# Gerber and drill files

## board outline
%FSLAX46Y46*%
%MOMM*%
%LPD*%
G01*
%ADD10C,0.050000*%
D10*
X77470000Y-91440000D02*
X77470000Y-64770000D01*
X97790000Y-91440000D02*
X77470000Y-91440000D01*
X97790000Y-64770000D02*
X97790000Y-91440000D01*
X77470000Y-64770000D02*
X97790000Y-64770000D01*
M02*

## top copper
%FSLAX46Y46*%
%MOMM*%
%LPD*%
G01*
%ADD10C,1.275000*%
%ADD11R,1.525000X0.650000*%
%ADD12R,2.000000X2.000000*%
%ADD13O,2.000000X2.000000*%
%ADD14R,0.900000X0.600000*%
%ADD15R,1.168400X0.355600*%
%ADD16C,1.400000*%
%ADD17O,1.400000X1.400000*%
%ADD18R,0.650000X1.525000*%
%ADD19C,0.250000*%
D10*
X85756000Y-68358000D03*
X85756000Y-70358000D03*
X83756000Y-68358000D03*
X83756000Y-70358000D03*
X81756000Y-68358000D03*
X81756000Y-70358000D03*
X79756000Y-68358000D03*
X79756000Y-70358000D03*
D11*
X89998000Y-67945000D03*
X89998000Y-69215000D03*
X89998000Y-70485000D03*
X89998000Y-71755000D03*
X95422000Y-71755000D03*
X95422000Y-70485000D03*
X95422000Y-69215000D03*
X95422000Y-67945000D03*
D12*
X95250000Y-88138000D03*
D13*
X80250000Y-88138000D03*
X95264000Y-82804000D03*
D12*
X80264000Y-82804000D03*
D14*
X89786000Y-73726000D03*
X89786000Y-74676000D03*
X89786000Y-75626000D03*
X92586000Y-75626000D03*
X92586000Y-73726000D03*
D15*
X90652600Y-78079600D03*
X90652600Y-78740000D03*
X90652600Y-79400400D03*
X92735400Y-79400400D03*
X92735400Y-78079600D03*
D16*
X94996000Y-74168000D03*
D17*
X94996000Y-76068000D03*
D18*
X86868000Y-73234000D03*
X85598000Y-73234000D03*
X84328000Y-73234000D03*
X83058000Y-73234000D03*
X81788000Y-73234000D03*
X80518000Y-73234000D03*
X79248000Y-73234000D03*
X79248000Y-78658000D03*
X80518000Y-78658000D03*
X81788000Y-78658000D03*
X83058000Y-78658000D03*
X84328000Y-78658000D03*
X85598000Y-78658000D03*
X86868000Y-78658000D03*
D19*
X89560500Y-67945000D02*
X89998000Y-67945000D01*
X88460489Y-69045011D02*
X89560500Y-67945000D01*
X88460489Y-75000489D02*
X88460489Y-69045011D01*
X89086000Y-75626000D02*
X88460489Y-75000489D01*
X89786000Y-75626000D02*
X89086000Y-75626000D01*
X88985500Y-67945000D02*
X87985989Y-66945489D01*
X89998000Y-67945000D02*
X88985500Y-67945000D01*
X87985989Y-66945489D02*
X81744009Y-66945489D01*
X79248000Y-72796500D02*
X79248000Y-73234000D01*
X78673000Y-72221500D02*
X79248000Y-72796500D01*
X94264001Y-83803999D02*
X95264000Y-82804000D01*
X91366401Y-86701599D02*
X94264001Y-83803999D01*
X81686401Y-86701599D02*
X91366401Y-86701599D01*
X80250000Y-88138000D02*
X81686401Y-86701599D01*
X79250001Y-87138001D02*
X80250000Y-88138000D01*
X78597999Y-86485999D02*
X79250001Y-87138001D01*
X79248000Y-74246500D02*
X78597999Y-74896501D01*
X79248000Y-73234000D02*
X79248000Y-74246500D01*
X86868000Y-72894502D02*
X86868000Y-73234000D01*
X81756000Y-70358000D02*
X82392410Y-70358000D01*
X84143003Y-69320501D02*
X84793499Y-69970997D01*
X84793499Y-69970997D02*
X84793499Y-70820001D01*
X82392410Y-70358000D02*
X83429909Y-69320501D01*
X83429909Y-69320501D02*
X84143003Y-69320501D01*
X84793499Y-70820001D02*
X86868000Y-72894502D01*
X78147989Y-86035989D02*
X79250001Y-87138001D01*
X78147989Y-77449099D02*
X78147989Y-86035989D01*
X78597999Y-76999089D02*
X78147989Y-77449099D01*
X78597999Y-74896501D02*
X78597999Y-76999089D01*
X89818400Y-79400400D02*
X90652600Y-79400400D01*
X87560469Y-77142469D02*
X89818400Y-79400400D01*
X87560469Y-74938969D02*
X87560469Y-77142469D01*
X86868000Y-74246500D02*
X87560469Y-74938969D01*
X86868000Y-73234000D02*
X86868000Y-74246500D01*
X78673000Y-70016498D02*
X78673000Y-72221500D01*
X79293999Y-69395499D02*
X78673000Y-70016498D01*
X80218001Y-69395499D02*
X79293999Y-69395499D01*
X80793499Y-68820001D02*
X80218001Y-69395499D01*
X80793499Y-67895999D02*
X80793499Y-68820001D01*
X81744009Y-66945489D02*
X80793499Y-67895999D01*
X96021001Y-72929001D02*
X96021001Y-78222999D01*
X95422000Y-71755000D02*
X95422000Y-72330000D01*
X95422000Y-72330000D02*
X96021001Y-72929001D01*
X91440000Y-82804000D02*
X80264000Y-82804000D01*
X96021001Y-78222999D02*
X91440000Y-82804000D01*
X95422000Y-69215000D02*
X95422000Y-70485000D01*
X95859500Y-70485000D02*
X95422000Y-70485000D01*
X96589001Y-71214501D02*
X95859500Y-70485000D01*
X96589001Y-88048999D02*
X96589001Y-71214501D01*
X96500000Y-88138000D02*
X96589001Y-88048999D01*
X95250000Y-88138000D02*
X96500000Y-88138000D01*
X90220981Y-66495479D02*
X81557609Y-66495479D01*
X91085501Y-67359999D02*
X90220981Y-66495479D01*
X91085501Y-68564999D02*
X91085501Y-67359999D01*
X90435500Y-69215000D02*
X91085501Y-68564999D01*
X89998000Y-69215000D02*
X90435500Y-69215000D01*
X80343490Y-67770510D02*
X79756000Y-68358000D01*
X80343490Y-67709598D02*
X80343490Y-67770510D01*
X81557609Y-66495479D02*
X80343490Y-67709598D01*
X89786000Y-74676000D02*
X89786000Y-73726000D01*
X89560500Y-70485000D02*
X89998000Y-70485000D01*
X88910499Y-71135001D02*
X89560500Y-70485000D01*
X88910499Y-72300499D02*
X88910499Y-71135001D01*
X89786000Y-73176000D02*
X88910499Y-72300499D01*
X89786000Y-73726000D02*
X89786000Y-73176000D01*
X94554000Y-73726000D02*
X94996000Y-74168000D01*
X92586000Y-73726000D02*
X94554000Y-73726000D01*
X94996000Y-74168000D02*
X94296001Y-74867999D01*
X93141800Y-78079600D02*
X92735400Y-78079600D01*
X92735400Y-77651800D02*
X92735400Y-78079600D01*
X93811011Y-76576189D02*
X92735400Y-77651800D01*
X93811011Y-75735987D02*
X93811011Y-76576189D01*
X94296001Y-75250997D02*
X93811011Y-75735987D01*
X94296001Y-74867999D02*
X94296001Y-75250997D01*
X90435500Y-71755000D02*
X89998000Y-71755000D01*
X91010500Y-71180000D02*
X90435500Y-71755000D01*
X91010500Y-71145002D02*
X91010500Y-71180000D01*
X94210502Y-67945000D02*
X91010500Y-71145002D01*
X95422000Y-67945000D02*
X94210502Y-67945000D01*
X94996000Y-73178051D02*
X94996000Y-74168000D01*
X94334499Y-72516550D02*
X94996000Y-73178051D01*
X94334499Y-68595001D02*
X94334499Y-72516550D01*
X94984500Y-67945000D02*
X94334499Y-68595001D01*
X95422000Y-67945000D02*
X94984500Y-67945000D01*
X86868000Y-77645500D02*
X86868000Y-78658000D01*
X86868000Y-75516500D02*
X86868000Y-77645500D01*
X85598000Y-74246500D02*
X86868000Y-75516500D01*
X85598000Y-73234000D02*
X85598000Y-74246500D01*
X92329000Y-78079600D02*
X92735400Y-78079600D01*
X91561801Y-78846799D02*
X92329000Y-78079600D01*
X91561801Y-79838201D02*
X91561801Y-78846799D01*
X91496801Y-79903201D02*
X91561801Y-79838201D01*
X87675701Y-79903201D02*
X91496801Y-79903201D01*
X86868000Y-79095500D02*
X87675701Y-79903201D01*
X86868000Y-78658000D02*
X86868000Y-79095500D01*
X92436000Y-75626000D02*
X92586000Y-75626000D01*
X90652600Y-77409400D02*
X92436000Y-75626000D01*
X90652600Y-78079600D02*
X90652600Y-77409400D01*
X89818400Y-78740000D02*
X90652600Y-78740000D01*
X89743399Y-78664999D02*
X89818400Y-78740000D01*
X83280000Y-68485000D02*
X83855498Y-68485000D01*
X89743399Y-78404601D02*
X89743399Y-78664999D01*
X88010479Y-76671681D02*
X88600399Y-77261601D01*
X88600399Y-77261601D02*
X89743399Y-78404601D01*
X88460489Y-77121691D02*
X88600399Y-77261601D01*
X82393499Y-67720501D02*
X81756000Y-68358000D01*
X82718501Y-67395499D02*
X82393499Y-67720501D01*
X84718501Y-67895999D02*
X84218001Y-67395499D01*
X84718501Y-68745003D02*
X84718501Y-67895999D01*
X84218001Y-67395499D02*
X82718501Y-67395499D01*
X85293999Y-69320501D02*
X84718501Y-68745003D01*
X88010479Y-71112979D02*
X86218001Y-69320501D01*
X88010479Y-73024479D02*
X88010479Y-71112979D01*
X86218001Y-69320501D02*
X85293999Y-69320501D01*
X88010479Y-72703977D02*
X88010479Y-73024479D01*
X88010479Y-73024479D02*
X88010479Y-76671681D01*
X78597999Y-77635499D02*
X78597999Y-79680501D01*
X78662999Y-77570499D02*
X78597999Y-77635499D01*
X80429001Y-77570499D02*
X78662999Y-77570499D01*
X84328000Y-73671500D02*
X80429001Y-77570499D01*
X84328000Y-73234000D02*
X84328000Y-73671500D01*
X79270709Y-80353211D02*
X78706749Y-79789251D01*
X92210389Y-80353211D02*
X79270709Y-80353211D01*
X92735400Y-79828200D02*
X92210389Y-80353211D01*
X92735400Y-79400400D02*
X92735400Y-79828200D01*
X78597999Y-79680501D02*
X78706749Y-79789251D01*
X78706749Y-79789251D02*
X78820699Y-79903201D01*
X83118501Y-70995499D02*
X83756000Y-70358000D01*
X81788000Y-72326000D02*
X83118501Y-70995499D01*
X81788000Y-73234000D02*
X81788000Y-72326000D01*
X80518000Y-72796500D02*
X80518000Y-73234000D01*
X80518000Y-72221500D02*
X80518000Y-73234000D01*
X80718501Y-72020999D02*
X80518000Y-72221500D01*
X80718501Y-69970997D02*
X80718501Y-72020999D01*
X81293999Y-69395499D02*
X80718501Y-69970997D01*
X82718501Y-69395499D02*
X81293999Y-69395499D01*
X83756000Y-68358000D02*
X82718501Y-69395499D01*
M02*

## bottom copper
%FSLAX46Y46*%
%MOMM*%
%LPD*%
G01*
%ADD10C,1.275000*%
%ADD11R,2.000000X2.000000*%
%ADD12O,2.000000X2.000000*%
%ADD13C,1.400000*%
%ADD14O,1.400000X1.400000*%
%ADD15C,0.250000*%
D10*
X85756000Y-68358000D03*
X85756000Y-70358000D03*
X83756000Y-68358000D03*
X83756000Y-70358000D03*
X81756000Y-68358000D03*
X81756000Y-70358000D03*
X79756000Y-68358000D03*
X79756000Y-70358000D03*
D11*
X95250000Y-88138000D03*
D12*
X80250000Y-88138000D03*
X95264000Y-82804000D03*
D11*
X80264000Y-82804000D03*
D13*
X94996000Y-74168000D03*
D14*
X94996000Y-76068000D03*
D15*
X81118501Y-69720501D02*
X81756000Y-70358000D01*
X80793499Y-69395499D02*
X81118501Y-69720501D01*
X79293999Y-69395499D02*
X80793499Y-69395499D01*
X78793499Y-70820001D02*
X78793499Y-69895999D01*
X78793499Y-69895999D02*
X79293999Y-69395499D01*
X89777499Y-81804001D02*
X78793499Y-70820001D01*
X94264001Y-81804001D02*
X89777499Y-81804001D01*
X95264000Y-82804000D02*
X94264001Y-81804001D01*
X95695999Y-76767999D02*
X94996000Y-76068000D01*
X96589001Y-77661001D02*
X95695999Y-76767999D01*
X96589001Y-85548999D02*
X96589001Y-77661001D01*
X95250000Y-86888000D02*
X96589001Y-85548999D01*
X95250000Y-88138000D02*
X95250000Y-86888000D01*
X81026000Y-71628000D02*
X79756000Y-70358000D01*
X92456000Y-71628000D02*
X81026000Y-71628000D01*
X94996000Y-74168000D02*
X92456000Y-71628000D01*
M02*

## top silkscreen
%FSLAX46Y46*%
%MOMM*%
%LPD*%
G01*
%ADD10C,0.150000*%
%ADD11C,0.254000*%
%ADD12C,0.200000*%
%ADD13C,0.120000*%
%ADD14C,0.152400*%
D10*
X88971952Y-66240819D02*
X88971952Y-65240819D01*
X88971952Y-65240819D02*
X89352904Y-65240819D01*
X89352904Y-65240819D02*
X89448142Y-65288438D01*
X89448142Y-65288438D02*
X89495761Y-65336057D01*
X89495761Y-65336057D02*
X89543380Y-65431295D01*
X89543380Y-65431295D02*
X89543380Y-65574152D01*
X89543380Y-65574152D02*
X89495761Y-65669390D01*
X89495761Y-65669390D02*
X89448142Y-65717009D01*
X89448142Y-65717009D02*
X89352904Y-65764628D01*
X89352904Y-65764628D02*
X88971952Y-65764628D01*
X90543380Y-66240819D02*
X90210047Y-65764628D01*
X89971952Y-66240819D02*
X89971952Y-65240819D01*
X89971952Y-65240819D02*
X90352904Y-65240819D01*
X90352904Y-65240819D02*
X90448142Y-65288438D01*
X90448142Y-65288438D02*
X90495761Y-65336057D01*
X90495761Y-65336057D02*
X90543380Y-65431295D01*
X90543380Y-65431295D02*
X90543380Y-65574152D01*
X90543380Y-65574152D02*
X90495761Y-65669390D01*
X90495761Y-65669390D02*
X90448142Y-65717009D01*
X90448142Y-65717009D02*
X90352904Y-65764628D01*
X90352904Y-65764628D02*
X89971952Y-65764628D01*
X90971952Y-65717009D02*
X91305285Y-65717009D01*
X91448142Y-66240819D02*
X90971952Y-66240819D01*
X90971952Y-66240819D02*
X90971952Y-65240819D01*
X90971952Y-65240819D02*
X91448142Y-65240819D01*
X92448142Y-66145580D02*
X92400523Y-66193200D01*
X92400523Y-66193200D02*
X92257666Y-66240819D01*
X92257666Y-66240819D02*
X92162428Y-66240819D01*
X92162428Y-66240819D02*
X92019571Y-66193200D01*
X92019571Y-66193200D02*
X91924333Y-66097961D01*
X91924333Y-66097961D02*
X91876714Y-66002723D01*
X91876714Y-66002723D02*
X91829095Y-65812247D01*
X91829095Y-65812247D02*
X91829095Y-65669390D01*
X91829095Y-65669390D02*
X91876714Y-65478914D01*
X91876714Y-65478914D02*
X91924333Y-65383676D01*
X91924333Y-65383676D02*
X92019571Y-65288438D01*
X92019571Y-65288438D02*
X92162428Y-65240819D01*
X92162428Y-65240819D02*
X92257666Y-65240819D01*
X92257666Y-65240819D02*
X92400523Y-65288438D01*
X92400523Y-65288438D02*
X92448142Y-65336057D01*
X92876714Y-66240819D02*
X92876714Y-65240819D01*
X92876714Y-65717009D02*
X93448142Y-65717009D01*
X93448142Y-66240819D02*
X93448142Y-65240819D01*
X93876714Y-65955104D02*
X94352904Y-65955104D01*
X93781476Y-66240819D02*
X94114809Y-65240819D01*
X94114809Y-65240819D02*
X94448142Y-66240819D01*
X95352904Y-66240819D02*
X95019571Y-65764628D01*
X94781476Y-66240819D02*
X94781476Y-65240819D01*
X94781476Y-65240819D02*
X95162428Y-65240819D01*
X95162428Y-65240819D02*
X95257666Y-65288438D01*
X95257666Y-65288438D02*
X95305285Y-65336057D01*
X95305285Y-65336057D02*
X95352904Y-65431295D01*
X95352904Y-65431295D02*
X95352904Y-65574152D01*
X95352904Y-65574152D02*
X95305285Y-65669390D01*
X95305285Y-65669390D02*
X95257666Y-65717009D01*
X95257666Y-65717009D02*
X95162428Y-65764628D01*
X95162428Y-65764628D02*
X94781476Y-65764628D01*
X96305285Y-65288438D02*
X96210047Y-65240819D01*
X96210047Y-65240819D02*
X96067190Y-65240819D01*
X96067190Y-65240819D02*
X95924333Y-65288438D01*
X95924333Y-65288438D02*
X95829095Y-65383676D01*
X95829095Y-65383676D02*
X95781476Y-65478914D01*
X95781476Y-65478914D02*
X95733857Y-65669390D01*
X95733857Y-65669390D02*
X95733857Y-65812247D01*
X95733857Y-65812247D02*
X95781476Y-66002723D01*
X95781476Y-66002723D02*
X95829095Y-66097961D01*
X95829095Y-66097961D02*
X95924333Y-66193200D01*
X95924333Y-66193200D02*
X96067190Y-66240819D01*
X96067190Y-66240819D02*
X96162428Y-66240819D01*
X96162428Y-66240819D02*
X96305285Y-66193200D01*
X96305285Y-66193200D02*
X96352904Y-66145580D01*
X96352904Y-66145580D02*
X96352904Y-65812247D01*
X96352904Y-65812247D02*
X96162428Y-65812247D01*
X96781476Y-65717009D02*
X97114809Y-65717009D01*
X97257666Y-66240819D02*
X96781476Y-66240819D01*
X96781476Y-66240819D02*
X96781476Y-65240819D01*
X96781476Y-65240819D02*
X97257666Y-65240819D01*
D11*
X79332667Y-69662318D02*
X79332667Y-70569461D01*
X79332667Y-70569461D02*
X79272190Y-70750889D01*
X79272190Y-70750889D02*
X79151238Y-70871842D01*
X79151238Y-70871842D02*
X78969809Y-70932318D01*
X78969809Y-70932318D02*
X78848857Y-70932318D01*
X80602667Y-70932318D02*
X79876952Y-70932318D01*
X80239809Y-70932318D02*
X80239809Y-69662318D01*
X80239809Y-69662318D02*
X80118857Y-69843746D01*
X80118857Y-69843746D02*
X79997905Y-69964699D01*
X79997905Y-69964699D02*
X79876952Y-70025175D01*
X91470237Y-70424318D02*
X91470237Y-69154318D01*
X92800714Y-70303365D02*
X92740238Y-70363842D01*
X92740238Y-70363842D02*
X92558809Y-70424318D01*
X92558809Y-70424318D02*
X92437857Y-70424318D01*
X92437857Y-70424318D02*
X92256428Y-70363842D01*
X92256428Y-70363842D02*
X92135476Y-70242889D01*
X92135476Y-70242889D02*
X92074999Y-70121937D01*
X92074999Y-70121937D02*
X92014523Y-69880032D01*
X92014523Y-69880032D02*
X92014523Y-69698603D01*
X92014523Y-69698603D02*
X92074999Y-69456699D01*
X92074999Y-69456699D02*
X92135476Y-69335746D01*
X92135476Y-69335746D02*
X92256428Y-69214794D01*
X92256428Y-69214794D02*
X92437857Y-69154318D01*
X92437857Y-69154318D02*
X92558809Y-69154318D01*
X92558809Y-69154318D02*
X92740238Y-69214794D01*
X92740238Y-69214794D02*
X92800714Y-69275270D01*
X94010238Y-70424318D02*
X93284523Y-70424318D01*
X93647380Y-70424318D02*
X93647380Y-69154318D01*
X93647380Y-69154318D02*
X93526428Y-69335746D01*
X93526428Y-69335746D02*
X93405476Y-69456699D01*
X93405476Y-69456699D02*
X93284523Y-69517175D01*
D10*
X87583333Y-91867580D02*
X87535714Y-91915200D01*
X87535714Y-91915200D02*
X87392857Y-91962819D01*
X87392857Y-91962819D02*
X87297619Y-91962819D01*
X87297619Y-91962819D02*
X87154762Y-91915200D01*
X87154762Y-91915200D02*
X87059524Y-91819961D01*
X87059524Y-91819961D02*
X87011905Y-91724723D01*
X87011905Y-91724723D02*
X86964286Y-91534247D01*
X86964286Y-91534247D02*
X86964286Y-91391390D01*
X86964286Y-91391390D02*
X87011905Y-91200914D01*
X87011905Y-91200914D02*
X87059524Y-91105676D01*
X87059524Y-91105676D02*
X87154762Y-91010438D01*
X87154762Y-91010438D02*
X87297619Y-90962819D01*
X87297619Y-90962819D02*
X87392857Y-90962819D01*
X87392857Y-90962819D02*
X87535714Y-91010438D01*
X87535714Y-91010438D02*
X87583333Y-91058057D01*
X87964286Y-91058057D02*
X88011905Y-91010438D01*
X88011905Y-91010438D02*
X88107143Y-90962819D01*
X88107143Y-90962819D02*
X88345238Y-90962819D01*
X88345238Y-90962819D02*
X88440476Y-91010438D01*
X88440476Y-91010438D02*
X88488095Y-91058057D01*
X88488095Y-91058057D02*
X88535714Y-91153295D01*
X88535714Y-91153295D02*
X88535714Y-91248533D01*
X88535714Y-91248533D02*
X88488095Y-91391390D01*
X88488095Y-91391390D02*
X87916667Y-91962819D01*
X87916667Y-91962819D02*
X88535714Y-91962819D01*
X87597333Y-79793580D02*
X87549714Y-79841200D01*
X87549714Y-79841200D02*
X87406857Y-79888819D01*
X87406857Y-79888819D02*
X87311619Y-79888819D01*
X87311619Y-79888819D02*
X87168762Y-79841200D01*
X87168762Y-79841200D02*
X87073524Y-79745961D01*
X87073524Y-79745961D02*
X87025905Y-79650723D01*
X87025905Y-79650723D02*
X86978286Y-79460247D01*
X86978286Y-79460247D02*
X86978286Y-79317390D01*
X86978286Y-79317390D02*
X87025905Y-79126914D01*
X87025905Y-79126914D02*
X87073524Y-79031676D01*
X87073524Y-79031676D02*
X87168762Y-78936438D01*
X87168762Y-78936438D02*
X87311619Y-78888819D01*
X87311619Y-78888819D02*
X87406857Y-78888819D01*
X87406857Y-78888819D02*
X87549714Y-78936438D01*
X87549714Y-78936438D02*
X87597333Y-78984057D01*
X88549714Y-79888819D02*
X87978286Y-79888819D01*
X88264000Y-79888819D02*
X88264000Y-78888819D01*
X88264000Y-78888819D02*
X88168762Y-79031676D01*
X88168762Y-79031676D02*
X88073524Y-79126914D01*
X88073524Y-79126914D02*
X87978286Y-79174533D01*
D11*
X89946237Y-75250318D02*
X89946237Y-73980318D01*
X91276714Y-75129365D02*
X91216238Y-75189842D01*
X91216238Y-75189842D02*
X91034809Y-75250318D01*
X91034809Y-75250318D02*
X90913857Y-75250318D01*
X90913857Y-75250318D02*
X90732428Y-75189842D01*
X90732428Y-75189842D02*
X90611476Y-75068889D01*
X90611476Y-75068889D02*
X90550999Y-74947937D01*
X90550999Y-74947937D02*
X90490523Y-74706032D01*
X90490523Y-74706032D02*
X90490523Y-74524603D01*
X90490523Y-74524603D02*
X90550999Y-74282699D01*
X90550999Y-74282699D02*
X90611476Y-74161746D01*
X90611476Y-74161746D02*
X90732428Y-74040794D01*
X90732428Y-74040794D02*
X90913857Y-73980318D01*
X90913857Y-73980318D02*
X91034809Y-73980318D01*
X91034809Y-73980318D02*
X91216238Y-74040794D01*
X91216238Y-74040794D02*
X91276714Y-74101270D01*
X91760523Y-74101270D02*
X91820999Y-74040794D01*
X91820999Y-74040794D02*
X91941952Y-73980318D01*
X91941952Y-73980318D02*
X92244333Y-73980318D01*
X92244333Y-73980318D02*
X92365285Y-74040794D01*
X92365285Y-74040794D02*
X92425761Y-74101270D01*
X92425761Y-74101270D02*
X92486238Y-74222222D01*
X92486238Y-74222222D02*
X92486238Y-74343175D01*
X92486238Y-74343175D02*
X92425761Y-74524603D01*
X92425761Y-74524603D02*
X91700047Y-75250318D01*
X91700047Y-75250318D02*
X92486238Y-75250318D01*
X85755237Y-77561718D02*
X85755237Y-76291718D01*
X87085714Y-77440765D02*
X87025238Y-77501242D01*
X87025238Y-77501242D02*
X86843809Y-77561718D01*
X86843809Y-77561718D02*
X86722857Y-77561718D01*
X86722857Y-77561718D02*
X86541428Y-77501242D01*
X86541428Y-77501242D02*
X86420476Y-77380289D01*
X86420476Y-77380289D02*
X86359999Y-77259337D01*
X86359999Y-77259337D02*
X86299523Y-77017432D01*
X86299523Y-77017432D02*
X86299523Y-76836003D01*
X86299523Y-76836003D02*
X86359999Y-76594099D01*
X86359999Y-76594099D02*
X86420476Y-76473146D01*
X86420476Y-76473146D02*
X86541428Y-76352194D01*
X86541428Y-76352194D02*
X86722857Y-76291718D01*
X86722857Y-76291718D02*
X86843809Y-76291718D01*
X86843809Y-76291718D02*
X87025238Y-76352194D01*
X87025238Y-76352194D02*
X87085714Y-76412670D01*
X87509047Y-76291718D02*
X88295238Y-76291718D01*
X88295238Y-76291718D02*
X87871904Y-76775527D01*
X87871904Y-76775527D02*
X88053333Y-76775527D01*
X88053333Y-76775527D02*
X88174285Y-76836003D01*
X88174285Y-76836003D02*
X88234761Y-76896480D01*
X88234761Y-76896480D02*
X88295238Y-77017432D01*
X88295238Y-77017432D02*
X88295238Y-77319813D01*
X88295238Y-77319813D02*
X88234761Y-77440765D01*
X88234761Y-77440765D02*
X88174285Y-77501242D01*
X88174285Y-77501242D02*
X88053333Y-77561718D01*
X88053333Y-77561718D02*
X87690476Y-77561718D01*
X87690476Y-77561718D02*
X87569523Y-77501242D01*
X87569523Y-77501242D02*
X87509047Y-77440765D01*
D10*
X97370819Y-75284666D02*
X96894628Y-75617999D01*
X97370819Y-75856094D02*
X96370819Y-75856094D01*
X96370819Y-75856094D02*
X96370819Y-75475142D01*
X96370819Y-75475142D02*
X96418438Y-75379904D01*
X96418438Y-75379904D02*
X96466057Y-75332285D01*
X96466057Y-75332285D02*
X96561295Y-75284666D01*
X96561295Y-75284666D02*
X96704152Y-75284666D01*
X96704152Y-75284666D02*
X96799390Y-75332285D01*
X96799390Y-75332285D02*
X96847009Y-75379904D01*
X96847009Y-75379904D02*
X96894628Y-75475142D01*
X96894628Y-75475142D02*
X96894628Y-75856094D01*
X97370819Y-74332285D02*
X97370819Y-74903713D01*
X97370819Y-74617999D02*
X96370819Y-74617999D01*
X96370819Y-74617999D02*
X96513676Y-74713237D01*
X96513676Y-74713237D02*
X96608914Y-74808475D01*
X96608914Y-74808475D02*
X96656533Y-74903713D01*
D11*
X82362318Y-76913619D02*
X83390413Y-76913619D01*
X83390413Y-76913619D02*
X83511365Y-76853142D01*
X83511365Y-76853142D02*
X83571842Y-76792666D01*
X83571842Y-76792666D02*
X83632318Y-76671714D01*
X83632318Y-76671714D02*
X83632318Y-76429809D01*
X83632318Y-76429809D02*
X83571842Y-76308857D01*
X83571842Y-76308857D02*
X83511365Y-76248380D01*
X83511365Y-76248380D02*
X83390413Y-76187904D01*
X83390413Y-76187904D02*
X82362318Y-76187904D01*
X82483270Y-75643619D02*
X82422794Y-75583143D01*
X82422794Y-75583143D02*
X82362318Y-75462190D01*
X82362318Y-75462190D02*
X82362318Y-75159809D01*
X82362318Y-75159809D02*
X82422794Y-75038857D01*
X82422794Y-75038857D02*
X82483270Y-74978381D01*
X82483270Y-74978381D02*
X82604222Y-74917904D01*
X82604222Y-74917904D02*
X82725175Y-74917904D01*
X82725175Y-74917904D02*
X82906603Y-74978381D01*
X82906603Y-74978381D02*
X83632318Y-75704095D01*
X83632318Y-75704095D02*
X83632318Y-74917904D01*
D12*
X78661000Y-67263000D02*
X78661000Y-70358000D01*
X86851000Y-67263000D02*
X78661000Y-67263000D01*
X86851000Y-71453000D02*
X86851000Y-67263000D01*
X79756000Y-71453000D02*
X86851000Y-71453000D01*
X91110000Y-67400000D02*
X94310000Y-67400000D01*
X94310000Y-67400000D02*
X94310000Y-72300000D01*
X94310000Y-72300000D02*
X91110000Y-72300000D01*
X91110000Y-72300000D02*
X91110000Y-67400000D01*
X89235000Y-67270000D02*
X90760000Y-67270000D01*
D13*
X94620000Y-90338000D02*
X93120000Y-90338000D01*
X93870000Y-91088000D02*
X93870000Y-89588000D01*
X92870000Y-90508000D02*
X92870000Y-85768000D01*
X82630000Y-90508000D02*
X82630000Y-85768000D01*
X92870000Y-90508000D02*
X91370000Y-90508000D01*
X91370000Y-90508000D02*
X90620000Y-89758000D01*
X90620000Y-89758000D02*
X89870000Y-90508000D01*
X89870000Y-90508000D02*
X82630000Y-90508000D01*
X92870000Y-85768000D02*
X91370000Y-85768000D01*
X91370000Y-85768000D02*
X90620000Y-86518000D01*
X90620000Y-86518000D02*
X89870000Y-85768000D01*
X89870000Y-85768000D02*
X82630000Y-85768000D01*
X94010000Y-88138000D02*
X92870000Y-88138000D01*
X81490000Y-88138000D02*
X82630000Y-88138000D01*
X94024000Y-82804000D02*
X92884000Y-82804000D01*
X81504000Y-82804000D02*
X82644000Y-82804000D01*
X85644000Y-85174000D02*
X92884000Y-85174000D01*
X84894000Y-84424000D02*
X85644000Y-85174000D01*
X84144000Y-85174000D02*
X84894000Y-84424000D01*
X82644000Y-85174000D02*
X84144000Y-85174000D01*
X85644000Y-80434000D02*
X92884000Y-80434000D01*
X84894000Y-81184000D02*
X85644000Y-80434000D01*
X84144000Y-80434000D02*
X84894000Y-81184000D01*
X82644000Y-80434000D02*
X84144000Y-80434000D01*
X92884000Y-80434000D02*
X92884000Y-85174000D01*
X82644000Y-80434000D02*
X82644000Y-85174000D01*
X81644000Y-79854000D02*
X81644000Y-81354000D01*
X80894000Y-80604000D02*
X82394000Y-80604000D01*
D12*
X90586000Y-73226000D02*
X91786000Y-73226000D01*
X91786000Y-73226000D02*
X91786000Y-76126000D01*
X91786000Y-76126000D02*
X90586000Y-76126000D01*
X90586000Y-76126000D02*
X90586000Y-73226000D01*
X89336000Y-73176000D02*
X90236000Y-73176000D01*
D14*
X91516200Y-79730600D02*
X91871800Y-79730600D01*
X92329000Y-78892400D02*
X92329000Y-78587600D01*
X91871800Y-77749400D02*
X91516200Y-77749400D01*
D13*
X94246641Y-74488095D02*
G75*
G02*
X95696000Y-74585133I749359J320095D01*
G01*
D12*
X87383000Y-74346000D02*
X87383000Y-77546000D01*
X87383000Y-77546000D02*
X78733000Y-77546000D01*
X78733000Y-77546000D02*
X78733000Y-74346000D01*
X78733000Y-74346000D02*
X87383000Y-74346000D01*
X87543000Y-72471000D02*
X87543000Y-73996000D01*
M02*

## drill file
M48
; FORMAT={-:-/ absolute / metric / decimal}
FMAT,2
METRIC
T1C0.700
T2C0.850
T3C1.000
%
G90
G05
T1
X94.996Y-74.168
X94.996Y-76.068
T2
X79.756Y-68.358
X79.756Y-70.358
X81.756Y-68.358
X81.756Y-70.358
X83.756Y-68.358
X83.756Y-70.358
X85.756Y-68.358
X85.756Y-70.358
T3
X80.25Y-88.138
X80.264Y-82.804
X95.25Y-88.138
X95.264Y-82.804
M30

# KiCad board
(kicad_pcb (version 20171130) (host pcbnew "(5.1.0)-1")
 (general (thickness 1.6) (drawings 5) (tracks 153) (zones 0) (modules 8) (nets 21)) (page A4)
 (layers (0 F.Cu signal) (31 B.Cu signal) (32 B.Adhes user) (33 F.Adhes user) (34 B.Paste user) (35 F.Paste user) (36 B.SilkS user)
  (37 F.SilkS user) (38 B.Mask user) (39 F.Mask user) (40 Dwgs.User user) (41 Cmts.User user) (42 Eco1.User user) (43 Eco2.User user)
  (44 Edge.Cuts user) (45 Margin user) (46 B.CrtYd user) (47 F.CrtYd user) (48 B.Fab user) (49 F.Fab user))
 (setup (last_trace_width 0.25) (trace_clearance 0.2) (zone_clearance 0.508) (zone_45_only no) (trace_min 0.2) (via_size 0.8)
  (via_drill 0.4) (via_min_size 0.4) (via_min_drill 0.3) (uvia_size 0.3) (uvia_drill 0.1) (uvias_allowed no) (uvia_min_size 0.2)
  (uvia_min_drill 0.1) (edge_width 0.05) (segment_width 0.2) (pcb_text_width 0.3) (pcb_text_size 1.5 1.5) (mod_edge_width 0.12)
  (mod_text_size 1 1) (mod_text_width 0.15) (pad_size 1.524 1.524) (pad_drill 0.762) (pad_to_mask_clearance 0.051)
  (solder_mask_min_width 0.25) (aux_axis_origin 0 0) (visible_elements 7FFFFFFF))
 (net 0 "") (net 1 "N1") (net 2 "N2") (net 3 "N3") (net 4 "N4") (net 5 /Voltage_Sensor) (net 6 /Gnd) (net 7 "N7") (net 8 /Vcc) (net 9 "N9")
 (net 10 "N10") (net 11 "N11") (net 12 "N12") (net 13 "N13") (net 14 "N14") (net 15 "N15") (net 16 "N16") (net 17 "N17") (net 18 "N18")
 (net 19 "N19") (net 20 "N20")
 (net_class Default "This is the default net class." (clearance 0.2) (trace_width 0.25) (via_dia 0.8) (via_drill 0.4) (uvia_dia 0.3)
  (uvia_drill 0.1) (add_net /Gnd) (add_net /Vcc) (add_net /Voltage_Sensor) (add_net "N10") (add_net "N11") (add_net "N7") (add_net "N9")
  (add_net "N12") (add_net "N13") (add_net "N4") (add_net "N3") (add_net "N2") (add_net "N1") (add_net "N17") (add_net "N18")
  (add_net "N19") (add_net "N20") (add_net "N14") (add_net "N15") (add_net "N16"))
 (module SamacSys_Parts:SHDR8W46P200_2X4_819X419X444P (layer F.Cu) (at 79.756 70.358)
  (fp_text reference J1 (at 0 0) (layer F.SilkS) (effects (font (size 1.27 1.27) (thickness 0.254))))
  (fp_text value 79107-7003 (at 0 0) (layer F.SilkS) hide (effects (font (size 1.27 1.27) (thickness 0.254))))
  (fp_line (start -1.095 -3.095) (end -1.095 0) (layer F.SilkS) (width 0.2))
  (fp_line (start 7.095 -3.095) (end -1.095 -3.095) (layer F.SilkS) (width 0.2))
  (fp_line (start 7.095 1.095) (end 7.095 -3.095) (layer F.SilkS) (width 0.2))
  (fp_line (start 0 1.095) (end 7.095 1.095) (layer F.SilkS) (width 0.2))
  (pad 8 thru_hole circle (at 6 -2) (size 1.275 1.275) (drill 0.85) (layers *.Cu *.Mask) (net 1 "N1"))
  (pad 7 thru_hole circle (at 6 0) (size 1.275 1.275) (drill 0.85) (layers *.Cu *.Mask) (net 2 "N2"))
  (pad 6 thru_hole circle (at 4 -2) (size 1.275 1.275) (drill 0.85) (layers *.Cu *.Mask) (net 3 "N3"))
  (pad 5 thru_hole circle (at 4 0) (size 1.275 1.275) (drill 0.85) (layers *.Cu *.Mask) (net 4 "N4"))
  (pad 4 thru_hole circle (at 2 -2) (size 1.275 1.275) (drill 0.85) (layers *.Cu *.Mask) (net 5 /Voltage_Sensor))
  (pad 3 thru_hole circle (at 2 0) (size 1.275 1.275) (drill 0.85) (layers *.Cu *.Mask) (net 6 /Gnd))
  (pad 2 thru_hole circle (at 0 -2) (size 1.275 1.275) (drill 0.85) (layers *.Cu *.Mask) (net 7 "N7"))
  (pad 1 thru_hole circle (at 0 0) (size 1.275 1.275) (drill 0.85) (layers *.Cu *.Mask) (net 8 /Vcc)))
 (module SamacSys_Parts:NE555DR (layer F.Cu) (at 92.71 69.85)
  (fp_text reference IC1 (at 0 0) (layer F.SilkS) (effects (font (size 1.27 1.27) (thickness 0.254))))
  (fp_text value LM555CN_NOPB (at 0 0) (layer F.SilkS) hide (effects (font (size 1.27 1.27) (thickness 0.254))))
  (fp_line (start -1.6 -2.45) (end 1.6 -2.45) (layer F.SilkS) (width 0.2))
  (fp_line (start 1.6 -2.45) (end 1.6 2.45) (layer F.SilkS) (width 0.2))
  (fp_line (start 1.6 2.45) (end -1.6 2.45) (layer F.SilkS) (width 0.2))
  (fp_line (start -1.6 2.45) (end -1.6 -2.45) (layer F.SilkS) (width 0.2))
  (fp_line (start -3.475 -2.58) (end -1.95 -2.58) (layer F.SilkS) (width 0.2))
  (pad 1 smd rect (at -2.712 -1.905 90) (size 0.65 1.525) (layers F.Cu F.Paste) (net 6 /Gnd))
  (pad 2 smd rect (at -2.712 -0.635 90) (size 0.65 1.525) (layers F.Cu F.Paste) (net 7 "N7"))
  (pad 3 smd rect (at -2.712 0.635 90) (size 0.65 1.525) (layers F.Cu F.Paste) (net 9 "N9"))
  (pad 4 smd rect (at -2.712 1.905 90) (size 0.65 1.525) (layers F.Cu F.Paste) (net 8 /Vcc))
  (pad 5 smd rect (at 2.712 1.905 90) (size 0.65 1.525) (layers F.Cu F.Paste) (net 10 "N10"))
  (pad 6 smd rect (at 2.712 0.635 90) (size 0.65 1.525) (layers F.Cu F.Paste) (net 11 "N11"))
  (pad 7 smd rect (at 2.712 -0.635 90) (size 0.65 1.525) (layers F.Cu F.Paste) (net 11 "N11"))
  (pad 8 smd rect (at 2.712 -1.905 90) (size 0.65 1.525) (layers F.Cu F.Paste) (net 8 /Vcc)))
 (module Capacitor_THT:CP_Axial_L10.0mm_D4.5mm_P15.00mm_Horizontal (layer F.Cu) (at 95.25 88.138 180)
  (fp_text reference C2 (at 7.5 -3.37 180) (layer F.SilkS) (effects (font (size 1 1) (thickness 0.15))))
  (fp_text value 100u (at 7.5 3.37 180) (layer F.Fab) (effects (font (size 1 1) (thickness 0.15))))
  (fp_line (start 0.63 -2.2) (end 2.13 -2.2) (layer F.SilkS) (width 0.12))
  (fp_line (start 1.38 -2.95) (end 1.38 -1.45) (layer F.SilkS) (width 0.12))
  (fp_line (start 2.38 -2.37) (end 2.38 2.37) (layer F.SilkS) (width 0.12))
  (fp_line (start 12.62 -2.37) (end 12.62 2.37) (layer F.SilkS) (width 0.12))
  (fp_line (start 2.38 -2.37) (end 3.88 -2.37) (layer F.SilkS) (width 0.12))
  (fp_line (start 3.88 -2.37) (end 4.63 -1.62) (layer F.SilkS) (width 0.12))
  (fp_line (start 4.63 -1.62) (end 5.38 -2.37) (layer F.SilkS) (width 0.12))
  (fp_line (start 5.38 -2.37) (end 12.62 -2.37) (layer F.SilkS) (width 0.12))
  (fp_line (start 2.38 2.37) (end 3.88 2.37) (layer F.SilkS) (width 0.12))
  (fp_line (start 3.88 2.37) (end 4.63 1.62) (layer F.SilkS) (width 0.12))
  (fp_line (start 4.63 1.62) (end 5.38 2.37) (layer F.SilkS) (width 0.12))
  (fp_line (start 5.38 2.37) (end 12.62 2.37) (layer F.SilkS) (width 0.12))
  (fp_line (start 1.24 0) (end 2.38 0) (layer F.SilkS) (width 0.12))
  (fp_line (start 13.76 0) (end 12.62 0) (layer F.SilkS) (width 0.12))
  (pad 1 thru_hole rect (at 0 0 180) (size 2 2) (drill 1) (layers *.Cu *.Mask) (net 11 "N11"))
  (pad 2 thru_hole oval (at 15 0 180) (size 2 2) (drill 1) (layers *.Cu *.Mask) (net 6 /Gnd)))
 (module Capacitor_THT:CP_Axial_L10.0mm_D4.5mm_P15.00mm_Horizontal (layer F.Cu) (at 80.264 82.804)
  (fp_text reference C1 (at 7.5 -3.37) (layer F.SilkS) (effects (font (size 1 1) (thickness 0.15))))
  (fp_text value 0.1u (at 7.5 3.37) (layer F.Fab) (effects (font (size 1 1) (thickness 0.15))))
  (fp_line (start 13.76 0) (end 12.62 0) (layer F.SilkS) (width 0.12))
  (fp_line (start 1.24 0) (end 2.38 0) (layer F.SilkS) (width 0.12))
  (fp_line (start 5.38 2.37) (end 12.62 2.37) (layer F.SilkS) (width 0.12))
  (fp_line (start 4.63 1.62) (end 5.38 2.37) (layer F.SilkS) (width 0.12))
  (fp_line (start 3.88 2.37) (end 4.63 1.62) (layer F.SilkS) (width 0.12))
  (fp_line (start 2.38 2.37) (end 3.88 2.37) (layer F.SilkS) (width 0.12))
  (fp_line (start 5.38 -2.37) (end 12.62 -2.37) (layer F.SilkS) (width 0.12))
  (fp_line (start 4.63 -1.62) (end 5.38 -2.37) (layer F.SilkS) (width 0.12))
  (fp_line (start 3.88 -2.37) (end 4.63 -1.62) (layer F.SilkS) (width 0.12))
  (fp_line (start 2.38 -2.37) (end 3.88 -2.37) (layer F.SilkS) (width 0.12))
  (fp_line (start 12.62 -2.37) (end 12.62 2.37) (layer F.SilkS) (width 0.12))
  (fp_line (start 2.38 -2.37) (end 2.38 2.37) (layer F.SilkS) (width 0.12))
  (fp_line (start 1.38 -2.95) (end 1.38 -1.45) (layer F.SilkS) (width 0.12))
  (fp_line (start 0.63 -2.2) (end 2.13 -2.2) (layer F.SilkS) (width 0.12))
  (pad 2 thru_hole oval (at 15 0) (size 2 2) (drill 1) (layers *.Cu *.Mask) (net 6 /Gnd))
  (pad 1 thru_hole rect (at 0 0) (size 2 2) (drill 1) (layers *.Cu *.Mask) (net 10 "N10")))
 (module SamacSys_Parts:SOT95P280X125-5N (layer F.Cu) (at 91.186 74.676)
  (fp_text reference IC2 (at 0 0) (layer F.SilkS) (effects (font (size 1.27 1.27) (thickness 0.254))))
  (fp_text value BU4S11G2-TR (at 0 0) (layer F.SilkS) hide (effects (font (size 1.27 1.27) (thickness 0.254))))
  (fp_line (start -0.6 -1.45) (end 0.6 -1.45) (layer F.SilkS) (width 0.2))
  (fp_line (start 0.6 -1.45) (end 0.6 1.45) (layer F.SilkS) (width 0.2))
  (fp_line (start 0.6 1.45) (end -0.6 1.45) (layer F.SilkS) (width 0.2))
  (fp_line (start -0.6 1.45) (end -0.6 -1.45) (layer F.SilkS) (width 0.2))
  (fp_line (start -1.85 -1.5) (end -0.95 -1.5) (layer F.SilkS) (width 0.2))
  (pad 1 smd rect (at -1.4 -0.95 90) (size 0.6 0.9) (layers F.Cu F.Paste F.Mask) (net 9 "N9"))
  (pad 2 smd rect (at -1.4 0 90) (size 0.6 0.9) (layers F.Cu F.Paste F.Mask) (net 9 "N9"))
  (pad 3 smd rect (at -1.4 0.95 90) (size 0.6 0.9) (layers F.Cu F.Paste F.Mask) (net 6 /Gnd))
  (pad 4 smd rect (at 1.4 0.95 90) (size 0.6 0.9) (layers F.Cu F.Paste F.Mask) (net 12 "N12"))
  (pad 5 smd rect (at 1.4 -0.95 90) (size 0.6 0.9) (layers F.Cu F.Paste F.Mask) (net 8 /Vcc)))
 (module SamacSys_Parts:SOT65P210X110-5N (layer F.Cu) (at 91.694 78.74)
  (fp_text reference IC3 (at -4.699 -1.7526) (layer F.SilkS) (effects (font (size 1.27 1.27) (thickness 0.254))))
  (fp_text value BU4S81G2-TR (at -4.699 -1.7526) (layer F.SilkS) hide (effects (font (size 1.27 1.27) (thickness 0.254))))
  (fp_line (start -0.1778 0.9906) (end 0.1778 0.9906) (layer F.SilkS) (width 0.1524))
  (fp_line (start 0.635 0.1524) (end 0.635 -0.1524) (layer F.SilkS) (width 0.1524))
  (fp_line (start 0.1778 -0.9906) (end -0.1778 -0.9906) (layer F.SilkS) (width 0.1524))
  (pad 1 smd rect (at -1.0414 -0.6604 90) (size 0.3556 1.1684) (layers F.Cu F.Paste F.Mask) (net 12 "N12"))
  (pad 2 smd rect (at -1.0414 0 90) (size 0.3556 1.1684) (layers F.Cu F.Paste F.Mask) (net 5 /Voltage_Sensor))
  (pad 3 smd rect (at -1.0414 0.6604 90) (size 0.3556 1.1684) (layers F.Cu F.Paste F.Mask) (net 6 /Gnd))
  (pad 4 smd rect (at 1.0414 0.6604 90) (size 0.3556 1.1684) (layers F.Cu F.Paste F.Mask) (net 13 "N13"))
  (pad 5 smd rect (at 1.0414 -0.6604 90) (size 0.3556 1.1684) (layers F.Cu F.Paste F.Mask) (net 8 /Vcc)))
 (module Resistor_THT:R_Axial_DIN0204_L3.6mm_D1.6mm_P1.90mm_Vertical (layer F.Cu) (at 94.996 74.168 270)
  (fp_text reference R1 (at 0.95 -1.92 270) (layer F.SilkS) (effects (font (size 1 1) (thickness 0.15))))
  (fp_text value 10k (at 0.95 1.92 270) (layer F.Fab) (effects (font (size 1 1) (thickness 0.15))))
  (fp_arc (start 0 0) (end 0.417133 -0.7) (angle -233.92106) (layer F.SilkS) (width 0.12))
  (pad 1 thru_hole circle (at 0 0 270) (size 1.4 1.4) (drill 0.7) (layers *.Cu *.Mask) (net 8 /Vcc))
  (pad 2 thru_hole oval (at 1.9 0 270) (size 1.4 1.4) (drill 0.7) (layers *.Cu *.Mask) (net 11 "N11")))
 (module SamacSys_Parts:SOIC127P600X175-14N (layer F.Cu) (at 83.058 75.946 270)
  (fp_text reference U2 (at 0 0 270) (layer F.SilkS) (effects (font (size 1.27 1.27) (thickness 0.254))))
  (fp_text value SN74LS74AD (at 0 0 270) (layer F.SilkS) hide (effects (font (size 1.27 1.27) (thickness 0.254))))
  (fp_line (start -1.6 -4.325) (end 1.6 -4.325) (layer F.SilkS) (width 0.2))
  (fp_line (start 1.6 -4.325) (end 1.6 4.325) (layer F.SilkS) (width 0.2))
  (fp_line (start 1.6 4.325) (end -1.6 4.325) (layer F.SilkS) (width 0.2))
  (fp_line (start -1.6 4.325) (end -1.6 -4.325) (layer F.SilkS) (width 0.2))
  (fp_line (start -3.475 -4.485) (end -1.95 -4.485) (layer F.SilkS) (width 0.2))
  (pad 1 smd rect (at -2.712 -3.81) (size 0.65 1.525) (layers F.Cu F.Paste F.Mask) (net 6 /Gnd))
  (pad 2 smd rect (at -2.712 -2.54) (size 0.65 1.525) (layers F.Cu F.Paste F.Mask) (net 8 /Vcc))
  (pad 3 smd rect (at -2.712 -1.27) (size 0.65 1.525) (layers F.Cu F.Paste F.Mask) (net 13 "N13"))
  (pad 4 smd rect (at -2.712 0) (size 0.65 1.525) (layers F.Cu F.Paste F.Mask) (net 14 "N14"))
  (pad 5 smd rect (at -2.712 1.27) (size 0.65 1.525) (layers F.Cu F.Paste F.Mask) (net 4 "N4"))
  (pad 6 smd rect (at -2.712 2.54) (size 0.65 1.525) (layers F.Cu F.Paste F.Mask) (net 3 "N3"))
  (pad 7 smd rect (at -2.712 3.81) (size 0.65 1.525) (layers F.Cu F.Paste F.Mask) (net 6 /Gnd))
  (pad 8 smd rect (at 2.712 3.81) (size 0.65 1.525) (layers F.Cu F.Paste F.Mask) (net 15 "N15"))
  (pad 9 smd rect (at 2.712 2.54) (size 0.65 1.525) (layers F.Cu F.Paste F.Mask) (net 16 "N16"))
  (pad 10 smd rect (at 2.712 1.27) (size 0.65 1.525) (layers F.Cu F.Paste F.Mask) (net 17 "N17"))
  (pad 11 smd rect (at 2.712 0) (size 0.65 1.525) (layers F.Cu F.Paste F.Mask) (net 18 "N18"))
  (pad 12 smd rect (at 2.712 -1.27) (size 0.65 1.525) (layers F.Cu F.Paste F.Mask) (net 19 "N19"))
  (pad 13 smd rect (at 2.712 -2.54) (size 0.65 1.525) (layers F.Cu F.Paste F.Mask) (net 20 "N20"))
  (pad 14 smd rect (at 2.712 -3.81) (size 0.65 1.525) (layers F.Cu F.Paste F.Mask) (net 8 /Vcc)))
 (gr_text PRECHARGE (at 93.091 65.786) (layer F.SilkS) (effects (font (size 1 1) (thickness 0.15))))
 (gr_line (start 77.47 91.44) (end 77.47 64.77) (layer Edge.Cuts) (width 0.05))
 (gr_line (start 97.79 91.44) (end 77.47 91.44) (layer Edge.Cuts) (width 0.05))
 (gr_line (start 97.79 64.77) (end 97.79 91.44) (layer Edge.Cuts) (width 0.05))
 (gr_line (start 77.47 64.77) (end 97.79 64.77) (layer Edge.Cuts) (width 0.05))
 (segment (start 89.5605 67.945) (end 89.998 67.945) (width 0.25) (layer F.Cu) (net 6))
 (segment (start 88.460489 69.045011) (end 89.5605 67.945) (width 0.25) (layer F.Cu) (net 6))
 (segment (start 88.460489 75.000489) (end 88.460489 69.045011) (width 0.25) (layer F.Cu) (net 6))
 (segment (start 89.086 75.626) (end 88.460489 75.000489) (width 0.25) (layer F.Cu) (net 6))
 (segment (start 89.786 75.626) (end 89.086 75.626) (width 0.25) (layer F.Cu) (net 6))
 (segment (start 88.9855 67.945) (end 87.985989 66.945489) (width 0.25) (layer F.Cu) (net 6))
 (segment (start 89.998 67.945) (end 88.9855 67.945) (width 0.25) (layer F.Cu) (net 6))
 (segment (start 87.985989 66.945489) (end 81.744009 66.945489) (width 0.25) (layer F.Cu) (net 6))
 (segment (start 79.248 72.7965) (end 79.248 73.234) (width 0.25) (layer F.Cu) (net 6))
 (segment (start 78.673 72.2215) (end 79.248 72.7965) (width 0.25) (layer F.Cu) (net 6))
 (segment (start 94.264001 83.803999) (end 95.264 82.804) (width 0.25) (layer F.Cu) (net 6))
 (segment (start 91.366401 86.701599) (end 94.264001 83.803999) (width 0.25) (layer F.Cu) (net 6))
 (segment (start 81.686401 86.701599) (end 91.366401 86.701599) (width 0.25) (layer F.Cu) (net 6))
 (segment (start 80.25 88.138) (end 81.686401 86.701599) (width 0.25) (layer F.Cu) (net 6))
 (segment (start 81.118501 69.720501) (end 81.756 70.358) (width 0.25) (layer B.Cu) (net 6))
 (segment (start 80.793499 69.395499) (end 81.118501 69.720501) (width 0.25) (layer B.Cu) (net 6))
 (segment (start 79.293999 69.395499) (end 80.793499 69.395499) (width 0.25) (layer B.Cu) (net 6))
 (segment (start 78.793499 70.820001) (end 78.793499 69.895999) (width 0.25) (layer B.Cu) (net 6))
 (segment (start 78.793499 69.895999) (end 79.293999 69.395499) (width 0.25) (layer B.Cu) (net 6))
 (segment (start 89.777499 81.804001) (end 78.793499 70.820001) (width 0.25) (layer B.Cu) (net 6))
 (segment (start 94.264001 81.804001) (end 89.777499 81.804001) (width 0.25) (layer B.Cu) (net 6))
 (segment (start 95.264 82.804) (end 94.264001 81.804001) (width 0.25) (layer B.Cu) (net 6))
 (segment (start 79.250001 87.138001) (end 80.25 88.138) (width 0.25) (layer F.Cu) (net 6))
 (segment (start 78.597999 86.485999) (end 79.250001 87.138001) (width 0.25) (layer F.Cu) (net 6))
 (segment (start 79.248 74.2465) (end 78.597999 74.896501) (width 0.25) (layer F.Cu) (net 6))
 (segment (start 79.248 73.234) (end 79.248 74.2465) (width 0.25) (layer F.Cu) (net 6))
 (segment (start 86.868 72.894502) (end 86.868 73.234) (width 0.25) (layer F.Cu) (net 6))
 (segment (start 81.756 70.358) (end 82.39241 70.358) (width 0.25) (layer F.Cu) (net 6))
 (segment (start 84.143003 69.320501) (end 84.793499 69.970997) (width 0.25) (layer F.Cu) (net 6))
 (segment (start 84.793499 69.970997) (end 84.793499 70.820001) (width 0.25) (layer F.Cu) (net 6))
 (segment (start 82.39241 70.358) (end 83.429909 69.320501) (width 0.25) (layer F.Cu) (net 6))
 (segment (start 83.429909 69.320501) (end 84.143003 69.320501) (width 0.25) (layer F.Cu) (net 6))
 (segment (start 84.793499 70.820001) (end 86.868 72.894502) (width 0.25) (layer F.Cu) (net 6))
 (segment (start 78.147989 86.035989) (end 79.250001 87.138001) (width 0.25) (layer F.Cu) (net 6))
 (segment (start 78.147989 77.449099) (end 78.147989 86.035989) (width 0.25) (layer F.Cu) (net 6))
 (segment (start 78.597999 76.999089) (end 78.147989 77.449099) (width 0.25) (layer F.Cu) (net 6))
 (segment (start 78.597999 74.896501) (end 78.597999 76.999089) (width 0.25) (layer F.Cu) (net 6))
 (segment (start 89.8184 79.4004) (end 90.6526 79.4004) (width 0.25) (layer F.Cu) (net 6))
 (segment (start 87.560469 77.142469) (end 89.8184 79.4004) (width 0.25) (layer F.Cu) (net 6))
 (segment (start 87.560469 74.938969) (end 87.560469 77.142469) (width 0.25) (layer F.Cu) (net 6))
 (segment (start 86.868 74.2465) (end 87.560469 74.938969) (width 0.25) (layer F.Cu) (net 6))
 (segment (start 86.868 73.234) (end 86.868 74.2465) (width 0.25) (layer F.Cu) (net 6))
 (segment (start 78.673 70.016498) (end 78.673 72.2215) (width 0.25) (layer F.Cu) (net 6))
 (segment (start 79.293999 69.395499) (end 78.673 70.016498) (width 0.25) (layer F.Cu) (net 6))
 (segment (start 80.218001 69.395499) (end 79.293999 69.395499) (width 0.25) (layer F.Cu) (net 6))
 (segment (start 80.793499 68.820001) (end 80.218001 69.395499) (width 0.25) (layer F.Cu) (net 6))
 (segment (start 80.793499 67.895999) (end 80.793499 68.820001) (width 0.25) (layer F.Cu) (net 6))
 (segment (start 81.744009 66.945489) (end 80.793499 67.895999) (width 0.25) (layer F.Cu) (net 6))
 (segment (start 96.021001 72.929001) (end 96.021001 78.222999) (width 0.25) (layer F.Cu) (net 10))
 (segment (start 95.422 71.755) (end 95.422 72.33) (width 0.25) (layer F.Cu) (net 10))
 (segment (start 95.422 72.33) (end 96.021001 72.929001) (width 0.25) (layer F.Cu) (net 10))
 (segment (start 91.44 82.804) (end 80.264 82.804) (width 0.25) (layer F.Cu) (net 10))
 (segment (start 96.021001 78.222999) (end 91.44 82.804) (width 0.25) (layer F.Cu) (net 10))
 (segment (start 95.422 69.215) (end 95.422 70.485) (width 0.25) (layer F.Cu) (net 11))
 (segment (start 95.695999 76.767999) (end 94.996 76.068) (width 0.25) (layer B.Cu) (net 11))
 (segment (start 96.589001 77.661001) (end 95.695999 76.767999) (width 0.25) (layer B.Cu) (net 11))
 (segment (start 96.589001 85.548999) (end 96.589001 77.661001) (width 0.25) (layer B.Cu) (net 11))
 (segment (start 95.25 86.888) (end 96.589001 85.548999) (width 0.25) (layer B.Cu) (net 11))
 (segment (start 95.25 88.138) (end 95.25 86.888) (width 0.25) (layer B.Cu) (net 11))
 (segment (start 95.8595 70.485) (end 95.422 70.485) (width 0.25) (layer F.Cu) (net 11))
 (segment (start 96.589001 71.214501) (end 95.8595 70.485) (width 0.25) (layer F.Cu) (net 11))
 (segment (start 96.589001 88.048999) (end 96.589001 71.214501) (width 0.25) (layer F.Cu) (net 11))
 (segment (start 96.5 88.138) (end 96.589001 88.048999) (width 0.25) (layer F.Cu) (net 11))
 (segment (start 95.25 88.138) (end 96.5 88.138) (width 0.25) (layer F.Cu) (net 11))
 (segment (start 90.220981 66.495479) (end 81.557609 66.495479) (width 0.25) (layer F.Cu) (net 7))
 (segment (start 91.085501 67.359999) (end 90.220981 66.495479) (width 0.25) (layer F.Cu) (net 7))
 (segment (start 91.085501 68.564999) (end 91.085501 67.359999) (width 0.25) (layer F.Cu) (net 7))
 (segment (start 90.4355 69.215) (end 91.085501 68.564999) (width 0.25) (layer F.Cu) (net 7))
 (segment (start 89.998 69.215) (end 90.4355 69.215) (width 0.25) (layer F.Cu) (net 7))
 (segment (start 80.34349 67.77051) (end 79.756 68.358) (width 0.25) (layer F.Cu) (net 7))
 (segment (start 80.34349 67.709598) (end 80.34349 67.77051) (width 0.25) (layer F.Cu) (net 7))
 (segment (start 81.557609 66.495479) (end 80.34349 67.709598) (width 0.25) (layer F.Cu) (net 7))
 (segment (start 89.786 74.676) (end 89.786 73.726) (width 0.25) (layer F.Cu) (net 9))
 (segment (start 89.5605 70.485) (end 89.998 70.485) (width 0.25) (layer F.Cu) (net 9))
 (segment (start 88.910499 71.135001) (end 89.5605 70.485) (width 0.25) (layer F.Cu) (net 9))
 (segment (start 88.910499 72.300499) (end 88.910499 71.135001) (width 0.25) (layer F.Cu) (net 9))
 (segment (start 89.786 73.176) (end 88.910499 72.300499) (width 0.25) (layer F.Cu) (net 9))
 (segment (start 89.786 73.726) (end 89.786 73.176) (width 0.25) (layer F.Cu) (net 9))
 (segment (start 94.554 73.726) (end 94.996 74.168) (width 0.25) (layer F.Cu) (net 8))
 (segment (start 92.586 73.726) (end 94.554 73.726) (width 0.25) (layer F.Cu) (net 8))
 (segment (start 94.996 74.168) (end 94.296001 74.867999) (width 0.25) (layer F.Cu) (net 8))
 (segment (start 93.1418 78.0796) (end 92.7354 78.0796) (width 0.25) (layer F.Cu) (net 8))
 (segment (start 92.7354 77.6518) (end 92.7354 78.0796) (width 0.25) (layer F.Cu) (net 8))
 (segment (start 93.811011 76.576189) (end 92.7354 77.6518) (width 0.25) (layer F.Cu) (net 8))
 (segment (start 93.811011 75.735987) (end 93.811011 76.576189) (width 0.25) (layer F.Cu) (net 8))
 (segment (start 94.296001 75.250997) (end 93.811011 75.735987) (width 0.25) (layer F.Cu) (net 8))
 (segment (start 94.296001 74.867999) (end 94.296001 75.250997) (width 0.25) (layer F.Cu) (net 8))
 (segment (start 90.4355 71.755) (end 89.998 71.755) (width 0.25) (layer F.Cu) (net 8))
 (segment (start 91.0105 71.18) (end 90.4355 71.755) (width 0.25) (layer F.Cu) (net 8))
 (segment (start 91.0105 71.145002) (end 91.0105 71.18) (width 0.25) (layer F.Cu) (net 8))
 (segment (start 94.210502 67.945) (end 91.0105 71.145002) (width 0.25) (layer F.Cu) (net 8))
 (segment (start 95.422 67.945) (end 94.210502 67.945) (width 0.25) (layer F.Cu) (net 8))
 (segment (start 81.026 71.628) (end 79.756 70.358) (width 0.25) (layer B.Cu) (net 8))
 (segment (start 92.456 71.628) (end 81.026 71.628) (width 0.25) (layer B.Cu) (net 8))
 (segment (start 94.996 74.168) (end 92.456 71.628) (width 0.25) (layer B.Cu) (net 8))
 (segment (start 94.996 73.178051) (end 94.996 74.168) (width 0.25) (layer F.Cu) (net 8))
 (segment (start 94.334499 72.51655) (end 94.996 73.178051) (width 0.25) (layer F.Cu) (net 8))
 (segment (start 94.334499 68.595001) (end 94.334499 72.51655) (width 0.25) (layer F.Cu) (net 8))
 (segment (start 94.9845 67.945) (end 94.334499 68.595001) (width 0.25) (layer F.Cu) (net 8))
 (segment (start 95.422 67.945) (end 94.9845 67.945) (width 0.25) (layer F.Cu) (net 8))
 (segment (start 86.868 77.6455) (end 86.868 78.658) (width 0.25) (layer F.Cu) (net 8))
 (segment (start 86.868 75.5165) (end 86.868 77.6455) (width 0.25) (layer F.Cu) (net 8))
 (segment (start 85.598 74.2465) (end 86.868 75.5165) (width 0.25) (layer F.Cu) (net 8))
 (segment (start 85.598 73.234) (end 85.598 74.2465) (width 0.25) (layer F.Cu) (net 8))
 (segment (start 92.329 78.0796) (end 92.7354 78.0796) (width 0.25) (layer F.Cu) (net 8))
 (segment (start 91.561801 78.846799) (end 92.329 78.0796) (width 0.25) (layer F.Cu) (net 8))
 (segment (start 91.561801 79.838201) (end 91.561801 78.846799) (width 0.25) (layer F.Cu) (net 8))
 (segment (start 91.496801 79.903201) (end 91.561801 79.838201) (width 0.25) (layer F.Cu) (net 8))
 (segment (start 87.675701 79.903201) (end 91.496801 79.903201) (width 0.25) (layer F.Cu) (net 8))
 (segment (start 86.868 79.0955) (end 87.675701 79.903201) (width 0.25) (layer F.Cu) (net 8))
 (segment (start 86.868 78.658) (end 86.868 79.0955) (width 0.25) (layer F.Cu) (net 8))
 (segment (start 92.436 75.626) (end 92.586 75.626) (width 0.25) (layer F.Cu) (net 12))
 (segment (start 90.6526 77.4094) (end 92.436 75.626) (width 0.25) (layer F.Cu) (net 12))
 (segment (start 90.6526 78.0796) (end 90.6526 77.4094) (width 0.25) (layer F.Cu) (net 12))
 (segment (start 89.8184 78.74) (end 90.6526 78.74) (width 0.25) (layer F.Cu) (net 5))
 (segment (start 89.743399 78.664999) (end 89.8184 78.74) (width 0.25) (layer F.Cu) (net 5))
 (segment (start 83.28 68.485) (end 83.855498 68.485) (width 0.25) (layer F.Cu) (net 3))
 (segment (start 89.743399 78.404601) (end 89.743399 78.664999) (width 0.25) (layer F.Cu) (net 5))
 (segment (start 88.010479 76.671681) (end 88.600399 77.261601) (width 0.25) (layer F.Cu) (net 5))
 (segment (start 88.600399 77.261601) (end 89.743399 78.404601) (width 0.25) (layer F.Cu) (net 5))
 (segment (start 88.460489 77.121691) (end 88.600399 77.261601) (width 0.25) (layer F.Cu) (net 5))
 (segment (start 82.393499 67.720501) (end 81.756 68.358) (width 0.25) (layer F.Cu) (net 5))
 (segment (start 82.718501 67.395499) (end 82.393499 67.720501) (width 0.25) (layer F.Cu) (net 5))
 (segment (start 84.718501 67.895999) (end 84.218001 67.395499) (width 0.25) (layer F.Cu) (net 5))
 (segment (start 84.718501 68.745003) (end 84.718501 67.895999) (width 0.25) (layer F.Cu) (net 5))
 (segment (start 84.218001 67.395499) (end 82.718501 67.395499) (width 0.25) (layer F.Cu) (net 5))
 (segment (start 85.293999 69.320501) (end 84.718501 68.745003) (width 0.25) (layer F.Cu) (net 5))
 (segment (start 88.010479 71.112979) (end 86.218001 69.320501) (width 0.25) (layer F.Cu) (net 5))
 (segment (start 88.010479 73.024479) (end 88.010479 71.112979) (width 0.25) (layer F.Cu) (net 5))
 (segment (start 86.218001 69.320501) (end 85.293999 69.320501) (width 0.25) (layer F.Cu) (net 5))
 (segment (start 88.010479 72.703977) (end 88.010479 73.024479) (width 0.25) (layer F.Cu) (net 5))
 (segment (start 88.010479 73.024479) (end 88.010479 76.671681) (width 0.25) (layer F.Cu) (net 5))
 (segment (start 78.597999 77.635499) (end 78.597999 79.680501) (width 0.25) (layer F.Cu) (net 13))
 (segment (start 78.662999 77.570499) (end 78.597999 77.635499) (width 0.25) (layer F.Cu) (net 13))
 (segment (start 80.429001 77.570499) (end 78.662999 77.570499) (width 0.25) (layer F.Cu) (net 13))
 (segment (start 84.328 73.6715) (end 80.429001 77.570499) (width 0.25) (layer F.Cu) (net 13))
 (segment (start 84.328 73.234) (end 84.328 73.6715) (width 0.25) (layer F.Cu) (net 13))
 (segment (start 79.270709 80.353211) (end 78.706749 79.789251) (width 0.25) (layer F.Cu) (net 13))
 (segment (start 92.210389 80.353211) (end 79.270709 80.353211) (width 0.25) (layer F.Cu) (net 13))
 (segment (start 92.7354 79.8282) (end 92.210389 80.353211) (width 0.25) (layer F.Cu) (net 13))
 (segment (start 92.7354 79.4004) (end 92.7354 79.8282) (width 0.25) (layer F.Cu) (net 13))
 (segment (start 78.597999 79.680501) (end 78.706749 79.789251) (width 0.25) (layer F.Cu) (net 13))
 (segment (start 78.706749 79.789251) (end 78.820699 79.903201) (width 0.25) (layer F.Cu) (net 13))
 (segment (start 83.118501 70.995499) (end 83.756 70.358) (width 0.25) (layer F.Cu) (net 4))
 (segment (start 81.788 72.326) (end 83.118501 70.995499) (width 0.25) (layer F.Cu) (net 4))
 (segment (start 81.788 73.234) (end 81.788 72.326) (width 0.25) (layer F.Cu) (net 4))
 (segment (start 80.518 72.7965) (end 80.518 73.234) (width 0.25) (layer F.Cu) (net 3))
 (segment (start 80.518 72.2215) (end 80.518 73.234) (width 0.25) (layer F.Cu) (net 3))
 (segment (start 80.718501 72.020999) (end 80.518 72.2215) (width 0.25) (layer F.Cu) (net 3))
 (segment (start 80.718501 69.970997) (end 80.718501 72.020999) (width 0.25) (layer F.Cu) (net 3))
 (segment (start 81.293999 69.395499) (end 80.718501 69.970997) (width 0.25) (layer F.Cu) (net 3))
 (segment (start 82.718501 69.395499) (end 81.293999 69.395499) (width 0.25) (layer F.Cu) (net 3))
 (segment (start 83.756 68.358) (end 82.718501 69.395499) (width 0.25) (layer F.Cu) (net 3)))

